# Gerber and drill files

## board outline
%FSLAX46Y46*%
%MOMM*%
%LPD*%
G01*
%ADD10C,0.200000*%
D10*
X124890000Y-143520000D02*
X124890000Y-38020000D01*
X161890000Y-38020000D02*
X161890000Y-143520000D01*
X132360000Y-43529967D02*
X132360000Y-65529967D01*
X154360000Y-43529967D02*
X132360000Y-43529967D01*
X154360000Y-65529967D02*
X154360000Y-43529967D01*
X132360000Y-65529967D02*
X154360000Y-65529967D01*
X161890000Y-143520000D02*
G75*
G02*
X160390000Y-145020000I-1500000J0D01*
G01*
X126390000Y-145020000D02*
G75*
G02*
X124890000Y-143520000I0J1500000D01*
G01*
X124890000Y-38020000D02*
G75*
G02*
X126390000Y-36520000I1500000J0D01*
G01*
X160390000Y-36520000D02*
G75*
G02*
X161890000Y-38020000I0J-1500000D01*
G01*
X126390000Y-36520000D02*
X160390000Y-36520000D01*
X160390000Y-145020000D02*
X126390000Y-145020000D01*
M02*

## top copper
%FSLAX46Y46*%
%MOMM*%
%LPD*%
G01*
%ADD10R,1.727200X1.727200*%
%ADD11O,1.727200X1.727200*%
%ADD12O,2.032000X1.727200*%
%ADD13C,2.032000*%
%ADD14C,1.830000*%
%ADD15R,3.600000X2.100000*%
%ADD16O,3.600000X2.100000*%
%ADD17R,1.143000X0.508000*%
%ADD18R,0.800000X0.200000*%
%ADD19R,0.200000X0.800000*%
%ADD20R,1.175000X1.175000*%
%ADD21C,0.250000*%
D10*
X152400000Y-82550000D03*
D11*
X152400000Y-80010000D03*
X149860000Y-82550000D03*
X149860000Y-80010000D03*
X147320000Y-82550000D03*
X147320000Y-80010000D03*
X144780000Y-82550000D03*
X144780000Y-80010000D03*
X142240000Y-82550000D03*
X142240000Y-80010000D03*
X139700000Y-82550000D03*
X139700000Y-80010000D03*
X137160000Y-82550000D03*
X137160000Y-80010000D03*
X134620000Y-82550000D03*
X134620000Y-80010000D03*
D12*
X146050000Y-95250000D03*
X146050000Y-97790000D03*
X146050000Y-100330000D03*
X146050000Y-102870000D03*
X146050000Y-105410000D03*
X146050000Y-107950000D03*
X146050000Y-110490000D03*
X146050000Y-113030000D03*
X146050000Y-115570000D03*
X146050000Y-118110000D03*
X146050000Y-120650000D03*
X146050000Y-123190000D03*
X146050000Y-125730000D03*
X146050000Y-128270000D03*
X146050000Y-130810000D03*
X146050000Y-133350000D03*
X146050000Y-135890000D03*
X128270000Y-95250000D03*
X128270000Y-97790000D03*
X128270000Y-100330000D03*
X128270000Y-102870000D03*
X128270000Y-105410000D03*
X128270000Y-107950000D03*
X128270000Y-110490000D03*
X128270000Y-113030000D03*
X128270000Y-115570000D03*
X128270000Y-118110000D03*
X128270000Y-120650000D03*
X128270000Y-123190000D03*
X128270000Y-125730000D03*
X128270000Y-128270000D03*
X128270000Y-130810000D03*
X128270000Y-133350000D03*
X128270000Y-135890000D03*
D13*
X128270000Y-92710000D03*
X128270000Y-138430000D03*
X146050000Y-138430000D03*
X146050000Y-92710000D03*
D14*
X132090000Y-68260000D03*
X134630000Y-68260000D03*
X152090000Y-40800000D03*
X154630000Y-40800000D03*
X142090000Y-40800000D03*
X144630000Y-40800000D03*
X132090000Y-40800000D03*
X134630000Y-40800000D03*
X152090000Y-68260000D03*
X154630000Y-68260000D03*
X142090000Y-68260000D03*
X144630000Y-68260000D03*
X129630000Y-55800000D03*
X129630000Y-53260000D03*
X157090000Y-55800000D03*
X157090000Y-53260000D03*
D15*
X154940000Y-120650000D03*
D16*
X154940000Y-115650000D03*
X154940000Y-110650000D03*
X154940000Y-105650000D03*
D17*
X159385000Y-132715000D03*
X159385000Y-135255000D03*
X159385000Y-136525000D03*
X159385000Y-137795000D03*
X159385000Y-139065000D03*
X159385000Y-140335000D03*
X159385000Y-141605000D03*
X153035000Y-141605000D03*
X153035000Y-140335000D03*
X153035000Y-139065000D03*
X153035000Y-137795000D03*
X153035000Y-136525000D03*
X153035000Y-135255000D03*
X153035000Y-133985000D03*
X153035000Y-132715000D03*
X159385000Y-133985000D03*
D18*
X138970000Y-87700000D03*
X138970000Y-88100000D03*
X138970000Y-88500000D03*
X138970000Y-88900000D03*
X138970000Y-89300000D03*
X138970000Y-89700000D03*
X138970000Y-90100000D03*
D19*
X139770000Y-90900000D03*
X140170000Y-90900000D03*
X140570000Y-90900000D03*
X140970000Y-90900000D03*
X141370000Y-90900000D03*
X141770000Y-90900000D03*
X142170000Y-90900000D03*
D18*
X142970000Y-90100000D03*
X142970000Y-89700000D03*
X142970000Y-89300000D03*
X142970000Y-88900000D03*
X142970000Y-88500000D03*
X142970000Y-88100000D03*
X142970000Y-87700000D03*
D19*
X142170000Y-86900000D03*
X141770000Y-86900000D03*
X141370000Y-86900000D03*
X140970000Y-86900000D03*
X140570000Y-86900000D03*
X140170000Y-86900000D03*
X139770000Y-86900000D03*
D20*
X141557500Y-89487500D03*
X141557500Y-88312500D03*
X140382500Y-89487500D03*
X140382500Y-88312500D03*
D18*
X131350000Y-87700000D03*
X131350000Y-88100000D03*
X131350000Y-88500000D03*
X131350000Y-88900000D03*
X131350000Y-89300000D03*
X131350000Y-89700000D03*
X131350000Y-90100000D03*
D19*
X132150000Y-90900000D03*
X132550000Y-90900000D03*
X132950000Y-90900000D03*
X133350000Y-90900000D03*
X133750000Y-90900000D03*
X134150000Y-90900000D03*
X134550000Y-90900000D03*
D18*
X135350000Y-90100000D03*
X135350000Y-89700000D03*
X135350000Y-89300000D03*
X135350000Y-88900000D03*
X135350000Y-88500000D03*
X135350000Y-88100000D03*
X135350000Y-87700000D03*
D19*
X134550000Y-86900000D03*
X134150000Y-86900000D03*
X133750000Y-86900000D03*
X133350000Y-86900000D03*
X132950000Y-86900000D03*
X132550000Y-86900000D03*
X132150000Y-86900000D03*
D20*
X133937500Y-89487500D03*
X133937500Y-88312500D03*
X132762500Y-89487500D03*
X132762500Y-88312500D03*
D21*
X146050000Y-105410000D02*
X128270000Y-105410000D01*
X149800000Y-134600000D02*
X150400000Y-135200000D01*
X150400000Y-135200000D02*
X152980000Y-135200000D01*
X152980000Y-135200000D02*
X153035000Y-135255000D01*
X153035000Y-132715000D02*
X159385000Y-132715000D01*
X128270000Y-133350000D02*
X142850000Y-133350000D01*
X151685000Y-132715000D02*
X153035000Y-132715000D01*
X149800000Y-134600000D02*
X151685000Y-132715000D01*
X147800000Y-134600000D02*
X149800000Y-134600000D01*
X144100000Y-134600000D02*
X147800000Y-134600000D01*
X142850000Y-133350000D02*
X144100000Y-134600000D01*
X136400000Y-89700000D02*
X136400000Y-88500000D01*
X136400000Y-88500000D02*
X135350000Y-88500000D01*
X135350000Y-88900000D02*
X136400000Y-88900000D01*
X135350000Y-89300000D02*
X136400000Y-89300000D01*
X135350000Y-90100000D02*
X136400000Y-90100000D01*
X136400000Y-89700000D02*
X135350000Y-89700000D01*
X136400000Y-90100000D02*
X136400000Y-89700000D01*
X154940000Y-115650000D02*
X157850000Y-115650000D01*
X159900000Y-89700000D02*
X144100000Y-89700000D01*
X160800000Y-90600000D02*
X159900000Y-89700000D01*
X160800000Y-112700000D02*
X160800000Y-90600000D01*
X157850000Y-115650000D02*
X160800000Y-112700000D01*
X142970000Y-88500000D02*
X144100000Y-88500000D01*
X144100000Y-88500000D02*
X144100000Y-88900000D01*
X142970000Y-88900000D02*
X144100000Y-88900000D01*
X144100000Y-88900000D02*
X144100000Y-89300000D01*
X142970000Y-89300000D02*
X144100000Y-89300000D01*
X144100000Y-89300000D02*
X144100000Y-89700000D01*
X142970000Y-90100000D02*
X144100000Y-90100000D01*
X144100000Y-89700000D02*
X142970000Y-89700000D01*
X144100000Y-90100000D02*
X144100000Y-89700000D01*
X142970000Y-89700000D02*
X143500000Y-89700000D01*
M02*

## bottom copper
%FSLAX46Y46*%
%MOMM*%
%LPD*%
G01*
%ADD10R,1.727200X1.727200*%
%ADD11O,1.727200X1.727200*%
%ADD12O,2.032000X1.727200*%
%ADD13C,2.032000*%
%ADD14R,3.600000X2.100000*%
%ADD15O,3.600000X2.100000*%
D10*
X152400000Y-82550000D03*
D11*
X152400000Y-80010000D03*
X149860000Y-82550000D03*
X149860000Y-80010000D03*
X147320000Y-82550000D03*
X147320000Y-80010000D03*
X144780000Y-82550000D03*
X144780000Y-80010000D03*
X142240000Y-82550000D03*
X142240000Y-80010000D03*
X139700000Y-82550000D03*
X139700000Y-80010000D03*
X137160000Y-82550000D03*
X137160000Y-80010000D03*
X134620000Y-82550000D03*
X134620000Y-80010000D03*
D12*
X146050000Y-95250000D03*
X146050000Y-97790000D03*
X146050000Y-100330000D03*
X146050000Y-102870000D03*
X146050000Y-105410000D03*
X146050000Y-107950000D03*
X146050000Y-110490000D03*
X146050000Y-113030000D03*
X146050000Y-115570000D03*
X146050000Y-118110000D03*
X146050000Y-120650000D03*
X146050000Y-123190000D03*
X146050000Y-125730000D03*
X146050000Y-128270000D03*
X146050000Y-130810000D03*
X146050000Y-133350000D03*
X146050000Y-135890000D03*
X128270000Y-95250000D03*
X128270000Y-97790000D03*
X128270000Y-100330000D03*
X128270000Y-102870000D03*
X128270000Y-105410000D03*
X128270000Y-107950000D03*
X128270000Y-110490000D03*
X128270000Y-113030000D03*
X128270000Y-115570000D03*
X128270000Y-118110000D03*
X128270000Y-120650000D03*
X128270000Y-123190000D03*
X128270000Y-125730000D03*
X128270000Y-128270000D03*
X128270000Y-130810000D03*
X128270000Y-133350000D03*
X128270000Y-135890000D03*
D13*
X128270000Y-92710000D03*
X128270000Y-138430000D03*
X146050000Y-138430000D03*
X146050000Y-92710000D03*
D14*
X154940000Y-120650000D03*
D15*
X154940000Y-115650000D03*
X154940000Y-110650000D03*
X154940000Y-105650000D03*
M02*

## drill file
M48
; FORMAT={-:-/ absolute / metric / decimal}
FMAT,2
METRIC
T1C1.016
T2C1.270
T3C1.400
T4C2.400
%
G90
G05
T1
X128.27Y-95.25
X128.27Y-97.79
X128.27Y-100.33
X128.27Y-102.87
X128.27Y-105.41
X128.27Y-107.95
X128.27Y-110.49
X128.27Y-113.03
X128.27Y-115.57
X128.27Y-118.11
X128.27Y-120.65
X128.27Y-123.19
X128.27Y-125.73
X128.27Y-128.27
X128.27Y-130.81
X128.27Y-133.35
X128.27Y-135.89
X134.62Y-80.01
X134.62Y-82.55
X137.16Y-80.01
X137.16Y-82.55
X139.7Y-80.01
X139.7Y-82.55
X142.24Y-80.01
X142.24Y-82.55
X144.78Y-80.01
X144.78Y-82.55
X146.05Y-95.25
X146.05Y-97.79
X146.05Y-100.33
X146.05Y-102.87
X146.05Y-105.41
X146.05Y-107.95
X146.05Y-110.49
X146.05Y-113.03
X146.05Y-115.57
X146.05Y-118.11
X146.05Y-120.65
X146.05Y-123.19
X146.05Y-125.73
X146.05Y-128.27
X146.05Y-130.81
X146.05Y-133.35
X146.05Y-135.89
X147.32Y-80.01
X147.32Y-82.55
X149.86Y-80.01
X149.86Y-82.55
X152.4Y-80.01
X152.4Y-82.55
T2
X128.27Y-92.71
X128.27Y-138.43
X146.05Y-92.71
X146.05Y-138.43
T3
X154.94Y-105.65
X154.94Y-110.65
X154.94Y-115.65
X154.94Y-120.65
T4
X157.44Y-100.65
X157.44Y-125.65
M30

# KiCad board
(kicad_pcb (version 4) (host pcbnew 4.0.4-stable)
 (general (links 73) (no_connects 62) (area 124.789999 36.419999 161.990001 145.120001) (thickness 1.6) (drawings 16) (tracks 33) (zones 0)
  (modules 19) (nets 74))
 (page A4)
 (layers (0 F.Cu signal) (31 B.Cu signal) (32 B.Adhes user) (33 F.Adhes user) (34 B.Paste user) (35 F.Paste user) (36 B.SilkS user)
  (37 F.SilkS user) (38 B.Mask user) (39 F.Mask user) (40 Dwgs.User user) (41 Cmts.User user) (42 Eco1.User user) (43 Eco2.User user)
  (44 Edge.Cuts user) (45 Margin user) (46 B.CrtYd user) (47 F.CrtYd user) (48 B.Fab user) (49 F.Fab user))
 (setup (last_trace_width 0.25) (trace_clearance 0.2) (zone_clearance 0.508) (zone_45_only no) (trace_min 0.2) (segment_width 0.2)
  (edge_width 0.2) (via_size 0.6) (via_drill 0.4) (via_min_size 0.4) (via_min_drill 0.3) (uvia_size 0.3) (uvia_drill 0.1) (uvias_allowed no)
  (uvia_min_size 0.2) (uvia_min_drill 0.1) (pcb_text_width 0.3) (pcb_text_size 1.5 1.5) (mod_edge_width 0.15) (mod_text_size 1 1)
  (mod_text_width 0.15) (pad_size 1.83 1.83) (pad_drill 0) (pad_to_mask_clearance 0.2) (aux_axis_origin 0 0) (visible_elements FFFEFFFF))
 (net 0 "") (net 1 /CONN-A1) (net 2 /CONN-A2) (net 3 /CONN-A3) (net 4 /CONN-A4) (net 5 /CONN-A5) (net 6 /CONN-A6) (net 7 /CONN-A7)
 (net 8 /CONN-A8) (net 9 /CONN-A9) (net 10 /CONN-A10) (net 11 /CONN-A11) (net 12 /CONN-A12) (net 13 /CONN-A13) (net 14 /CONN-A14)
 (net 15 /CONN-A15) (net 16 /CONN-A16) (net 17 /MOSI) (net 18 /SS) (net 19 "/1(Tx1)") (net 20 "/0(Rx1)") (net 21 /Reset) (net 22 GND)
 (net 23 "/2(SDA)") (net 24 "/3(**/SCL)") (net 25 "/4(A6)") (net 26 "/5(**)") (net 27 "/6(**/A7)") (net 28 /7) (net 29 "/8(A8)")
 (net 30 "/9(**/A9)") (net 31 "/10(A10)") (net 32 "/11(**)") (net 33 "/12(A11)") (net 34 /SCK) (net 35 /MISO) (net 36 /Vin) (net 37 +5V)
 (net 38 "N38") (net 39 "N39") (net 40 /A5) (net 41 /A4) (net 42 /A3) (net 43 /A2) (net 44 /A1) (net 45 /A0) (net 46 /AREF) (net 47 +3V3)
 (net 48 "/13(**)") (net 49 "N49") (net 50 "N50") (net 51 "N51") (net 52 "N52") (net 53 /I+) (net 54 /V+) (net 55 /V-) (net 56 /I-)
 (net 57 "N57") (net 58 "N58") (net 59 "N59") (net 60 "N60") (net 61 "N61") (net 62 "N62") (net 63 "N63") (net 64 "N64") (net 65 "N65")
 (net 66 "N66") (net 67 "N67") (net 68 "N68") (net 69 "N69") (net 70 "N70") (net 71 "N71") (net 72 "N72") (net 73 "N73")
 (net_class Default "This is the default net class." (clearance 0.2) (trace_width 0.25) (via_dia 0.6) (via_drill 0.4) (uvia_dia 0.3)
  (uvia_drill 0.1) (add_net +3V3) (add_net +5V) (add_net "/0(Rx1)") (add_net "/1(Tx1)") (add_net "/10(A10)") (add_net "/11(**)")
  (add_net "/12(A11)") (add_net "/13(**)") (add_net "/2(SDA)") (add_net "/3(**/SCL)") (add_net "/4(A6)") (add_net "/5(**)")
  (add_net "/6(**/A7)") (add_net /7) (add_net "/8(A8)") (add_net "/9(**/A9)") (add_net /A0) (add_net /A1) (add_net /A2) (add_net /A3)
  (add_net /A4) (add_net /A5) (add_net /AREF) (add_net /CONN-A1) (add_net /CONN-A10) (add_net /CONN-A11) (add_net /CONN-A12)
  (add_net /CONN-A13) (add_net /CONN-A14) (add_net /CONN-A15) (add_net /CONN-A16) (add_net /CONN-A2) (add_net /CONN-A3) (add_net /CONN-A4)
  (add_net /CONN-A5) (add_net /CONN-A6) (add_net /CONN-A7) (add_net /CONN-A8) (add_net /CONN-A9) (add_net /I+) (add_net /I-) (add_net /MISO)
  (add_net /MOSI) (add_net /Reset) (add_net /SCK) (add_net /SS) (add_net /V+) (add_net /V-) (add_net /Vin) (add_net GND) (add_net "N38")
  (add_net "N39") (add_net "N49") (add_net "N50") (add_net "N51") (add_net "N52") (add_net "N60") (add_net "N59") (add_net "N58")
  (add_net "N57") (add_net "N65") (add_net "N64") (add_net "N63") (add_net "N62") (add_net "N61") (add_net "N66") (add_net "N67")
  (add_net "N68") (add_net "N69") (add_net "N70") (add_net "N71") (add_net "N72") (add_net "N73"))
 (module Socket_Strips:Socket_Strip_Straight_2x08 (layer F.Cu) (at 152.4 82.55 180)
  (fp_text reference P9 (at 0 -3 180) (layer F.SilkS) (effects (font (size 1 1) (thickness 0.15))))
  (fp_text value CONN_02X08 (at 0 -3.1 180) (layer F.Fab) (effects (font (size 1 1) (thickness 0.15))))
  (pad 1 thru_hole rect (at 0 0 180) (size 1.7272 1.7272) (drill 1.016) (layers *.Cu *.Mask F.SilkS) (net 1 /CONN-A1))
  (pad 2 thru_hole oval (at 0 2.54 180) (size 1.7272 1.7272) (drill 1.016) (layers *.Cu *.Mask F.SilkS) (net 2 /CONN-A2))
  (pad 3 thru_hole oval (at 2.54 0 180) (size 1.7272 1.7272) (drill 1.016) (layers *.Cu *.Mask F.SilkS) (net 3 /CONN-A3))
  (pad 4 thru_hole oval (at 2.54 2.54 180) (size 1.7272 1.7272) (drill 1.016) (layers *.Cu *.Mask F.SilkS) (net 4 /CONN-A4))
  (pad 5 thru_hole oval (at 5.08 0 180) (size 1.7272 1.7272) (drill 1.016) (layers *.Cu *.Mask F.SilkS) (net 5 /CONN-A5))
  (pad 6 thru_hole oval (at 5.08 2.54 180) (size 1.7272 1.7272) (drill 1.016) (layers *.Cu *.Mask F.SilkS) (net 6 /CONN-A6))
  (pad 7 thru_hole oval (at 7.62 0 180) (size 1.7272 1.7272) (drill 1.016) (layers *.Cu *.Mask F.SilkS) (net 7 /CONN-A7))
  (pad 8 thru_hole oval (at 7.62 2.54 180) (size 1.7272 1.7272) (drill 1.016) (layers *.Cu *.Mask F.SilkS) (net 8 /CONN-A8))
  (pad 9 thru_hole oval (at 10.16 0 180) (size 1.7272 1.7272) (drill 1.016) (layers *.Cu *.Mask F.SilkS) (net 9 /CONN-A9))
  (pad 10 thru_hole oval (at 10.16 2.54 180) (size 1.7272 1.7272) (drill 1.016) (layers *.Cu *.Mask F.SilkS) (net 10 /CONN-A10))
  (pad 11 thru_hole oval (at 12.7 0 180) (size 1.7272 1.7272) (drill 1.016) (layers *.Cu *.Mask F.SilkS) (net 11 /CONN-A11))
  (pad 12 thru_hole oval (at 12.7 2.54 180) (size 1.7272 1.7272) (drill 1.016) (layers *.Cu *.Mask F.SilkS) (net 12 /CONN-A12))
  (pad 13 thru_hole oval (at 15.24 0 180) (size 1.7272 1.7272) (drill 1.016) (layers *.Cu *.Mask F.SilkS) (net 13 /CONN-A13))
  (pad 14 thru_hole oval (at 15.24 2.54 180) (size 1.7272 1.7272) (drill 1.016) (layers *.Cu *.Mask F.SilkS) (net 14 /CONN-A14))
  (pad 15 thru_hole oval (at 17.78 0 180) (size 1.7272 1.7272) (drill 1.016) (layers *.Cu *.Mask F.SilkS) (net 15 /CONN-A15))
  (pad 16 thru_hole oval (at 17.78 2.54 180) (size 1.7272 1.7272) (drill 1.016) (layers *.Cu *.Mask F.SilkS) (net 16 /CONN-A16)))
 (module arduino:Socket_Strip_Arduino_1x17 (layer F.Cu) (at 146.05 95.25 270)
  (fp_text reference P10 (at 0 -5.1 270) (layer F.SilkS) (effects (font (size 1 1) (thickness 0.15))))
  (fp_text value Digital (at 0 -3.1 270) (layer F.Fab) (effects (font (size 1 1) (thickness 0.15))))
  (pad 1 thru_hole oval (at 0 0 270) (size 1.7272 2.032) (drill 1.016) (layers *.Cu *.Mask F.SilkS) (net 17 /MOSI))
  (pad 2 thru_hole oval (at 2.54 0 270) (size 1.7272 2.032) (drill 1.016) (layers *.Cu *.Mask F.SilkS) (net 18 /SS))
  (pad 3 thru_hole oval (at 5.08 0 270) (size 1.7272 2.032) (drill 1.016) (layers *.Cu *.Mask F.SilkS) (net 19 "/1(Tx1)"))
  (pad 4 thru_hole oval (at 7.62 0 270) (size 1.7272 2.032) (drill 1.016) (layers *.Cu *.Mask F.SilkS) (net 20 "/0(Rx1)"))
  (pad 5 thru_hole oval (at 10.16 0 270) (size 1.7272 2.032) (drill 1.016) (layers *.Cu *.Mask F.SilkS) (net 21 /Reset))
  (pad 6 thru_hole oval (at 12.7 0 270) (size 1.7272 2.032) (drill 1.016) (layers *.Cu *.Mask F.SilkS) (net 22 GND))
  (pad 7 thru_hole oval (at 15.24 0 270) (size 1.7272 2.032) (drill 1.016) (layers *.Cu *.Mask F.SilkS) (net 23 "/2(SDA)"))
  (pad 8 thru_hole oval (at 17.78 0 270) (size 1.7272 2.032) (drill 1.016) (layers *.Cu *.Mask F.SilkS) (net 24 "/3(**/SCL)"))
  (pad 9 thru_hole oval (at 20.32 0 270) (size 1.7272 2.032) (drill 1.016) (layers *.Cu *.Mask F.SilkS) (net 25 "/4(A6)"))
  (pad 10 thru_hole oval (at 22.86 0 270) (size 1.7272 2.032) (drill 1.016) (layers *.Cu *.Mask F.SilkS) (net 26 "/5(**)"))
  (pad 11 thru_hole oval (at 25.4 0 270) (size 1.7272 2.032) (drill 1.016) (layers *.Cu *.Mask F.SilkS) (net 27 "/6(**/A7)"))
  (pad 12 thru_hole oval (at 27.94 0 270) (size 1.7272 2.032) (drill 1.016) (layers *.Cu *.Mask F.SilkS) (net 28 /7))
  (pad 13 thru_hole oval (at 30.48 0 270) (size 1.7272 2.032) (drill 1.016) (layers *.Cu *.Mask F.SilkS) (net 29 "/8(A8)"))
  (pad 14 thru_hole oval (at 33.02 0 270) (size 1.7272 2.032) (drill 1.016) (layers *.Cu *.Mask F.SilkS) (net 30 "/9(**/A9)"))
  (pad 15 thru_hole oval (at 35.56 0 270) (size 1.7272 2.032) (drill 1.016) (layers *.Cu *.Mask F.SilkS) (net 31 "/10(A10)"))
  (pad 16 thru_hole oval (at 38.1 0 270) (size 1.7272 2.032) (drill 1.016) (layers *.Cu *.Mask F.SilkS) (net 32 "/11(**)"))
  (pad 17 thru_hole oval (at 40.64 0 270) (size 1.7272 2.032) (drill 1.016) (layers *.Cu *.Mask F.SilkS) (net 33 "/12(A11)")))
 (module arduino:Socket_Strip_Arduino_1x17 (layer F.Cu) (at 128.27 95.25 270)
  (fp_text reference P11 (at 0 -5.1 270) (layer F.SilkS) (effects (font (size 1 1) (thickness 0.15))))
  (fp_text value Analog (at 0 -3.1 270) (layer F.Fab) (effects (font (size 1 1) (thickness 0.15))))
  (pad 1 thru_hole oval (at 0 0 270) (size 1.7272 2.032) (drill 1.016) (layers *.Cu *.Mask F.SilkS) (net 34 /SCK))
  (pad 2 thru_hole oval (at 2.54 0 270) (size 1.7272 2.032) (drill 1.016) (layers *.Cu *.Mask F.SilkS) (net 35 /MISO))
  (pad 3 thru_hole oval (at 5.08 0 270) (size 1.7272 2.032) (drill 1.016) (layers *.Cu *.Mask F.SilkS) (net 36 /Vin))
  (pad 4 thru_hole oval (at 7.62 0 270) (size 1.7272 2.032) (drill 1.016) (layers *.Cu *.Mask F.SilkS) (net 22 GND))
  (pad 5 thru_hole oval (at 10.16 0 270) (size 1.7272 2.032) (drill 1.016) (layers *.Cu *.Mask F.SilkS) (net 21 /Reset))
  (pad 6 thru_hole oval (at 12.7 0 270) (size 1.7272 2.032) (drill 1.016) (layers *.Cu *.Mask F.SilkS) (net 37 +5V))
  (pad 7 thru_hole oval (at 15.24 0 270) (size 1.7272 2.032) (drill 1.016) (layers *.Cu *.Mask F.SilkS) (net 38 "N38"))
  (pad 8 thru_hole oval (at 17.78 0 270) (size 1.7272 2.032) (drill 1.016) (layers *.Cu *.Mask F.SilkS) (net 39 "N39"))
  (pad 9 thru_hole oval (at 20.32 0 270) (size 1.7272 2.032) (drill 1.016) (layers *.Cu *.Mask F.SilkS) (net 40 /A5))
  (pad 10 thru_hole oval (at 22.86 0 270) (size 1.7272 2.032) (drill 1.016) (layers *.Cu *.Mask F.SilkS) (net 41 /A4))
  (pad 11 thru_hole oval (at 25.4 0 270) (size 1.7272 2.032) (drill 1.016) (layers *.Cu *.Mask F.SilkS) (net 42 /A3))
  (pad 12 thru_hole oval (at 27.94 0 270) (size 1.7272 2.032) (drill 1.016) (layers *.Cu *.Mask F.SilkS) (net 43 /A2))
  (pad 13 thru_hole oval (at 30.48 0 270) (size 1.7272 2.032) (drill 1.016) (layers *.Cu *.Mask F.SilkS) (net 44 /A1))
  (pad 14 thru_hole oval (at 33.02 0 270) (size 1.7272 2.032) (drill 1.016) (layers *.Cu *.Mask F.SilkS) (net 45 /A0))
  (pad 15 thru_hole oval (at 35.56 0 270) (size 1.7272 2.032) (drill 1.016) (layers *.Cu *.Mask F.SilkS) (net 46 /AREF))
  (pad 16 thru_hole oval (at 38.1 0 270) (size 1.7272 2.032) (drill 1.016) (layers *.Cu *.Mask F.SilkS) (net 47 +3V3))
  (pad 17 thru_hole oval (at 40.64 0 270) (size 1.7272 2.032) (drill 1.016) (layers *.Cu *.Mask F.SilkS) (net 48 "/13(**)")))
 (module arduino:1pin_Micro (layer F.Cu) (at 128.27 92.71)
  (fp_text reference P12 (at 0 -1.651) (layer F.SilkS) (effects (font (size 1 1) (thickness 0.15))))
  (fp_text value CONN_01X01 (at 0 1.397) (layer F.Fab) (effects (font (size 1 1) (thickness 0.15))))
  (pad 1 thru_hole circle (at 0 0) (size 2.032 2.032) (drill 1.27) (layers *.Cu *.Mask F.SilkS) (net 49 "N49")))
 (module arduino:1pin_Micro (layer F.Cu) (at 128.27 138.43)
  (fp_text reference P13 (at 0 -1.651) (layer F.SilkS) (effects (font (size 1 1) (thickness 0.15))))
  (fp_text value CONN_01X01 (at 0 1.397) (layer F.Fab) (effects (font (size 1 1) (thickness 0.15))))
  (pad 1 thru_hole circle (at 0 0) (size 2.032 2.032) (drill 1.27) (layers *.Cu *.Mask F.SilkS) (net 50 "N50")))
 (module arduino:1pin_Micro (layer F.Cu) (at 146.05 138.43)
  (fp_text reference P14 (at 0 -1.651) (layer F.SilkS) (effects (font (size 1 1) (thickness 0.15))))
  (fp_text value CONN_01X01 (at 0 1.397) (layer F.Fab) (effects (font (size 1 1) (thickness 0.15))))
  (pad 1 thru_hole circle (at 0 0) (size 2.032 2.032) (drill 1.27) (layers *.Cu *.Mask F.SilkS) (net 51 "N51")))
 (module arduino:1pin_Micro (layer F.Cu) (at 146.05 92.71)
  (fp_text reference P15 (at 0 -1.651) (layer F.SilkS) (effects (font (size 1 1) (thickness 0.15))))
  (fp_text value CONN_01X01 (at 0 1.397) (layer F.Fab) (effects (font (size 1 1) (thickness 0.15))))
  (pad 1 thru_hole circle (at 0 0) (size 2.032 2.032) (drill 1.27) (layers *.Cu *.Mask F.SilkS) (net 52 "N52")))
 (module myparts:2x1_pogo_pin (layer F.Cu) (at 132.09 68.26)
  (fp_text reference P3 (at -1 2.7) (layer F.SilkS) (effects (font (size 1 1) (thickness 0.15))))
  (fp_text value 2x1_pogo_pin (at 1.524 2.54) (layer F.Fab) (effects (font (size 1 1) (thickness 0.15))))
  (pad 1 smd circle (at 0 0) (size 1.83 1.83) (layers F.Cu F.Paste F.Mask) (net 13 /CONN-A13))
  (pad 2 smd circle (at 2.54 0) (size 1.83 1.83) (layers F.Cu F.Paste F.Mask) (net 14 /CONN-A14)))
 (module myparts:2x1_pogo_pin (layer F.Cu) (at 152.09 40.8)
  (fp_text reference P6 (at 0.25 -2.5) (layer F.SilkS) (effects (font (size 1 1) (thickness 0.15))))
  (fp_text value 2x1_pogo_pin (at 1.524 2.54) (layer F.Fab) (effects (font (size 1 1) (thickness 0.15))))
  (pad 1 smd circle (at 0 0) (size 1.83 1.83) (layers F.Cu F.Paste F.Mask) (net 5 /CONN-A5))
  (pad 2 smd circle (at 2.54 0) (size 1.83 1.83) (layers F.Cu F.Paste F.Mask) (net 6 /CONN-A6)))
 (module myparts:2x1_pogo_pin (layer F.Cu) (at 142.09 40.8)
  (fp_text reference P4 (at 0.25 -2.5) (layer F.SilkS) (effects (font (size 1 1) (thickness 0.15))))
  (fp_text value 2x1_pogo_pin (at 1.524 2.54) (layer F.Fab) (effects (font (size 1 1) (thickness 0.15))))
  (pad 1 smd circle (at 0 0) (size 1.83 1.83) (layers F.Cu F.Paste F.Mask) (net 7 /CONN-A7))
  (pad 2 smd circle (at 2.54 0) (size 1.83 1.83) (layers F.Cu F.Paste F.Mask) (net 8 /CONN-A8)))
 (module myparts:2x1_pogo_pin (layer F.Cu) (at 132.09 40.8)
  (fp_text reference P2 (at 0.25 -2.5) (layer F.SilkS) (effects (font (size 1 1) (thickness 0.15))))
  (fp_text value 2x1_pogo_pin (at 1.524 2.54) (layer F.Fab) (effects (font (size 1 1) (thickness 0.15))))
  (pad 1 smd circle (at 0 0) (size 1.83 1.83) (layers F.Cu F.Paste F.Mask) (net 11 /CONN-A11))
  (pad 2 smd circle (at 2.54 0) (size 1.83 1.83) (layers F.Cu F.Paste F.Mask) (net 12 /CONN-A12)))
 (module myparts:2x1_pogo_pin (layer F.Cu) (at 152.09 68.26)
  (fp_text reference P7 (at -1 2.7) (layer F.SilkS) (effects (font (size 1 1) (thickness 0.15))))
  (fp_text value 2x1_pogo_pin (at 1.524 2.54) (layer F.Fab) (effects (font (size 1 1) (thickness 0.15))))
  (pad 1 smd circle (at 0 0) (size 1.83 1.83) (layers F.Cu F.Paste F.Mask) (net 3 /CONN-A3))
  (pad 2 smd circle (at 2.54 0) (size 1.83 1.83) (layers F.Cu F.Paste F.Mask) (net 4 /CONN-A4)))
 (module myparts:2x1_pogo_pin (layer F.Cu) (at 142.09 68.26)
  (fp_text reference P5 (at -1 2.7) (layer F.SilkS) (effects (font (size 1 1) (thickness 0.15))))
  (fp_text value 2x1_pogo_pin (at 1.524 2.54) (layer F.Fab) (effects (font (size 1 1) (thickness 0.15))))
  (pad 1 smd circle (at 0 0) (size 1.83 1.83) (layers F.Cu F.Paste F.Mask) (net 9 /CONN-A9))
  (pad 2 smd circle (at 2.54 0) (size 1.83 1.83) (layers F.Cu F.Paste F.Mask) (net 10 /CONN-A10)))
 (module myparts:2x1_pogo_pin (layer F.Cu) (at 129.63 55.8 90)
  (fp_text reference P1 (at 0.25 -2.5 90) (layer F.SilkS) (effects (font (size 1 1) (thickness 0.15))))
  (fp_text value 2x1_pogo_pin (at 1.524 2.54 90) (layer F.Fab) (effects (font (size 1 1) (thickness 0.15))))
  (pad 1 smd circle (at 0 0 90) (size 1.83 1.83) (layers F.Cu F.Paste F.Mask) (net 15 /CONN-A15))
  (pad 2 smd circle (at 2.54 0 90) (size 1.83 1.83) (layers F.Cu F.Paste F.Mask) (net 16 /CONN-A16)))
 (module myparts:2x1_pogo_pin (layer F.Cu) (at 157.09 55.8 90)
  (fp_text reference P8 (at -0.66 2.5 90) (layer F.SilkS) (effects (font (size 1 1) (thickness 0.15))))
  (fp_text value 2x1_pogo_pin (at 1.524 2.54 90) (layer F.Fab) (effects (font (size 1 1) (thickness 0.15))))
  (pad 1 smd circle (at 0 0 90) (size 1.83 1.83) (layers F.Cu F.Paste F.Mask) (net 1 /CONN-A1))
  (pad 2 smd circle (at 2.54 0 90) (size 1.83 1.83) (layers F.Cu F.Paste F.Mask) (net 2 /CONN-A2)))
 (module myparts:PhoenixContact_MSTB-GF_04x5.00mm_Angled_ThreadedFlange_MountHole (layer F.Cu) (at 154.94 120.65 90)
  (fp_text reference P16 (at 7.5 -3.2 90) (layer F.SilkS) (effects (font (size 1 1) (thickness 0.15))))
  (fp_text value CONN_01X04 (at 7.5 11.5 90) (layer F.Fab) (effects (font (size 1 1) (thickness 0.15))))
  (pad 1 thru_hole rect (at 0 0 90) (size 2.1 3.6) (drill 1.4) (layers *.Cu *.Mask) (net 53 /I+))
  (pad 2 thru_hole oval (at 5 0 90) (size 2.1 3.6) (drill 1.4) (layers *.Cu *.Mask) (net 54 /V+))
  (pad 3 thru_hole oval (at 10 0 90) (size 2.1 3.6) (drill 1.4) (layers *.Cu *.Mask) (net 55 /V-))
  (pad 4 thru_hole oval (at 15 0 90) (size 2.1 3.6) (drill 1.4) (layers *.Cu *.Mask) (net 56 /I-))
  (pad "" np_thru_hole circle (at -5 2.5 90) (size 2.4 2.4) (drill 2.4) (layers *.Cu *.Mask))
  (pad "" np_thru_hole circle (at 20 2.5 90) (size 2.4 2.4) (drill 2.4) (layers *.Cu *.Mask)))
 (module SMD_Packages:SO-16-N (layer F.Cu) (at 156.21 137.16 270)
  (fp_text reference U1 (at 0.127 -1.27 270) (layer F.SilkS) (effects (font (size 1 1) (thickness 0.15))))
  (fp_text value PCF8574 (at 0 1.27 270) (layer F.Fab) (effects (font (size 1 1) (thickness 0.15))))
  (pad 16 smd rect (at -4.445 -3.175 270) (size 0.508 1.143) (layers F.Cu F.Paste F.Mask) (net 47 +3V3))
  (pad 14 smd rect (at -1.905 -3.175 270) (size 0.508 1.143) (layers F.Cu F.Paste F.Mask) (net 24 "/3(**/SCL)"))
  (pad 13 smd rect (at -0.635 -3.175 270) (size 0.508 1.143) (layers F.Cu F.Paste F.Mask) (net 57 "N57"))
  (pad 12 smd rect (at 0.635 -3.175 270) (size 0.508 1.143) (layers F.Cu F.Paste F.Mask) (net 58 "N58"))
  (pad 11 smd rect (at 1.905 -3.175 270) (size 0.508 1.143) (layers F.Cu F.Paste F.Mask) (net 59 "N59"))
  (pad 10 smd rect (at 3.175 -3.175 270) (size 0.508 1.143) (layers F.Cu F.Paste F.Mask) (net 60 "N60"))
  (pad 9 smd rect (at 4.445 -3.175 270) (size 0.508 1.143) (layers F.Cu F.Paste F.Mask) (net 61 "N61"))
  (pad 8 smd rect (at 4.445 3.175 270) (size 0.508 1.143) (layers F.Cu F.Paste F.Mask) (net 22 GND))
  (pad 7 smd rect (at 3.175 3.175 270) (size 0.508 1.143) (layers F.Cu F.Paste F.Mask) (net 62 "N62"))
  (pad 6 smd rect (at 1.905 3.175 270) (size 0.508 1.143) (layers F.Cu F.Paste F.Mask) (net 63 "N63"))
  (pad 5 smd rect (at 0.635 3.175 270) (size 0.508 1.143) (layers F.Cu F.Paste F.Mask) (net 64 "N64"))
  (pad 4 smd rect (at -0.635 3.175 270) (size 0.508 1.143) (layers F.Cu F.Paste F.Mask) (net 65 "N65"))
  (pad 3 smd rect (at -1.905 3.175 270) (size 0.508 1.143) (layers F.Cu F.Paste F.Mask) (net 47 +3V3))
  (pad 2 smd rect (at -3.175 3.175 270) (size 0.508 1.143) (layers F.Cu F.Paste F.Mask) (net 22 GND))
  (pad 1 smd rect (at -4.445 3.175 270) (size 0.508 1.143) (layers F.Cu F.Paste F.Mask) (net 47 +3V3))
  (pad 15 smd rect (at -3.175 -3.175 270) (size 0.508 1.143) (layers F.Cu F.Paste F.Mask) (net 23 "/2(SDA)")))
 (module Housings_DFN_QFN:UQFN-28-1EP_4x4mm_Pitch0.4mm (layer F.Cu) (at 140.97 88.9)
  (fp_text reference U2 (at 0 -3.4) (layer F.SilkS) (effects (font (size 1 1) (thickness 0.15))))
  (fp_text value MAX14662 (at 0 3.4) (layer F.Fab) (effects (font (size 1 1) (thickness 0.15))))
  (pad 1 smd rect (at -2 -1.2) (size 0.8 0.2) (layers F.Cu F.Paste F.Mask) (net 47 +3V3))
  (pad 2 smd rect (at -2 -0.8) (size 0.8 0.2) (layers F.Cu F.Paste F.Mask) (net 16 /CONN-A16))
  (pad 3 smd rect (at -2 -0.4) (size 0.8 0.2) (layers F.Cu F.Paste F.Mask) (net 14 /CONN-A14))
  (pad 4 smd rect (at -2 0) (size 0.8 0.2) (layers F.Cu F.Paste F.Mask) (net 12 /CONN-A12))
  (pad 5 smd rect (at -2 0.4) (size 0.8 0.2) (layers F.Cu F.Paste F.Mask) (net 10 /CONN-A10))
  (pad 6 smd rect (at -2 0.8) (size 0.8 0.2) (layers F.Cu F.Paste F.Mask) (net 8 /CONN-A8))
  (pad 7 smd rect (at -2 1.2) (size 0.8 0.2) (layers F.Cu F.Paste F.Mask) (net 6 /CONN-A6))
  (pad 8 smd rect (at -1.2 2 90) (size 0.8 0.2) (layers F.Cu F.Paste F.Mask) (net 4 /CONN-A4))
  (pad 9 smd rect (at -0.8 2 90) (size 0.8 0.2) (layers F.Cu F.Paste F.Mask) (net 2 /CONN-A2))
  (pad 10 smd rect (at -0.4 2 90) (size 0.8 0.2) (layers F.Cu F.Paste F.Mask) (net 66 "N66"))
  (pad 11 smd rect (at 0 2 90) (size 0.8 0.2) (layers F.Cu F.Paste F.Mask) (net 22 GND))
  (pad 12 smd rect (at 0.4 2 90) (size 0.8 0.2) (layers F.Cu F.Paste F.Mask) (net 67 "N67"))
  (pad 13 smd rect (at 0.8 2 90) (size 0.8 0.2) (layers F.Cu F.Paste F.Mask) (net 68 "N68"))
  (pad 14 smd rect (at 1.2 2 90) (size 0.8 0.2) (layers F.Cu F.Paste F.Mask) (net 55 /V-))
  (pad 15 smd rect (at 2 1.2) (size 0.8 0.2) (layers F.Cu F.Paste F.Mask) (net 54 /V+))
  (pad 16 smd rect (at 2 0.8) (size 0.8 0.2) (layers F.Cu F.Paste F.Mask) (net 54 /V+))
  (pad 17 smd rect (at 2 0.4) (size 0.8 0.2) (layers F.Cu F.Paste F.Mask) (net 54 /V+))
  (pad 18 smd rect (at 2 0) (size 0.8 0.2) (layers F.Cu F.Paste F.Mask) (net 54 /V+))
  (pad 19 smd rect (at 2 -0.4) (size 0.8 0.2) (layers F.Cu F.Paste F.Mask) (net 54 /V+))
  (pad 20 smd rect (at 2 -0.8) (size 0.8 0.2) (layers F.Cu F.Paste F.Mask) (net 54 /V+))
  (pad 21 smd rect (at 2 -1.2) (size 0.8 0.2) (layers F.Cu F.Paste F.Mask) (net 55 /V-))
  (pad 22 smd rect (at 1.2 -2 90) (size 0.8 0.2) (layers F.Cu F.Paste F.Mask) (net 47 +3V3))
  (pad 23 smd rect (at 0.8 -2 90) (size 0.8 0.2) (layers F.Cu F.Paste F.Mask) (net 65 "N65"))
  (pad 24 smd rect (at 0.4 -2 90) (size 0.8 0.2) (layers F.Cu F.Paste F.Mask) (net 34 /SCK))
  (pad 25 smd rect (at 0 -2 90) (size 0.8 0.2) (layers F.Cu F.Paste F.Mask) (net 22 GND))
  (pad 26 smd rect (at -0.4 -2 90) (size 0.8 0.2) (layers F.Cu F.Paste F.Mask) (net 47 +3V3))
  (pad 27 smd rect (at -0.8 -2 90) (size 0.8 0.2) (layers F.Cu F.Paste F.Mask) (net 17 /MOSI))
  (pad 28 smd rect (at -1.2 -2 90) (size 0.8 0.2) (layers F.Cu F.Paste F.Mask) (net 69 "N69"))
  (pad 29 smd rect (at 0.5875 0.5875) (size 1.175 1.175) (layers F.Cu F.Paste F.Mask) (solder_paste_margin_ratio -0.2))
  (pad 29 smd rect (at 0.5875 -0.5875) (size 1.175 1.175) (layers F.Cu F.Paste F.Mask) (solder_paste_margin_ratio -0.2))
  (pad 29 smd rect (at -0.5875 0.5875) (size 1.175 1.175) (layers F.Cu F.Paste F.Mask) (solder_paste_margin_ratio -0.2))
  (pad 29 smd rect (at -0.5875 -0.5875) (size 1.175 1.175) (layers F.Cu F.Paste F.Mask) (solder_paste_margin_ratio -0.2)))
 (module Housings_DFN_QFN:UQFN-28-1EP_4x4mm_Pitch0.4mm (layer F.Cu) (at 133.35 88.9)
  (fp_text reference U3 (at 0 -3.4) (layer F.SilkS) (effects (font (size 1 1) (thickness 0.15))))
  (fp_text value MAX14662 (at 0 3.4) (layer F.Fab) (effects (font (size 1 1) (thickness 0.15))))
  (pad 1 smd rect (at -2 -1.2) (size 0.8 0.2) (layers F.Cu F.Paste F.Mask) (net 47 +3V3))
  (pad 2 smd rect (at -2 -0.8) (size 0.8 0.2) (layers F.Cu F.Paste F.Mask) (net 15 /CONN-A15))
  (pad 3 smd rect (at -2 -0.4) (size 0.8 0.2) (layers F.Cu F.Paste F.Mask) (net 13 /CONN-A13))
  (pad 4 smd rect (at -2 0) (size 0.8 0.2) (layers F.Cu F.Paste F.Mask) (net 11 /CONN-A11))
  (pad 5 smd rect (at -2 0.4) (size 0.8 0.2) (layers F.Cu F.Paste F.Mask) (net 9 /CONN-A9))
  (pad 6 smd rect (at -2 0.8) (size 0.8 0.2) (layers F.Cu F.Paste F.Mask) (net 7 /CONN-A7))
  (pad 7 smd rect (at -2 1.2) (size 0.8 0.2) (layers F.Cu F.Paste F.Mask) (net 5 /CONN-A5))
  (pad 8 smd rect (at -1.2 2 90) (size 0.8 0.2) (layers F.Cu F.Paste F.Mask) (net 3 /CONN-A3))
  (pad 9 smd rect (at -0.8 2 90) (size 0.8 0.2) (layers F.Cu F.Paste F.Mask) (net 1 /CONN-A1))
  (pad 10 smd rect (at -0.4 2 90) (size 0.8 0.2) (layers F.Cu F.Paste F.Mask) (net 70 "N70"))
  (pad 11 smd rect (at 0 2 90) (size 0.8 0.2) (layers F.Cu F.Paste F.Mask) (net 22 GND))
  (pad 12 smd rect (at 0.4 2 90) (size 0.8 0.2) (layers F.Cu F.Paste F.Mask) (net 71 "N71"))
  (pad 13 smd rect (at 0.8 2 90) (size 0.8 0.2) (layers F.Cu F.Paste F.Mask) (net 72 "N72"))
  (pad 14 smd rect (at 1.2 2 90) (size 0.8 0.2) (layers F.Cu F.Paste F.Mask) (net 56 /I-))
  (pad 15 smd rect (at 2 1.2) (size 0.8 0.2) (layers F.Cu F.Paste F.Mask) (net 53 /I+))
  (pad 16 smd rect (at 2 0.8) (size 0.8 0.2) (layers F.Cu F.Paste F.Mask) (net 53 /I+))
  (pad 17 smd rect (at 2 0.4) (size 0.8 0.2) (layers F.Cu F.Paste F.Mask) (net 53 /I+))
  (pad 18 smd rect (at 2 0) (size 0.8 0.2) (layers F.Cu F.Paste F.Mask) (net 53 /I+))
  (pad 19 smd rect (at 2 -0.4) (size 0.8 0.2) (layers F.Cu F.Paste F.Mask) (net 53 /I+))
  (pad 20 smd rect (at 2 -0.8) (size 0.8 0.2) (layers F.Cu F.Paste F.Mask) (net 53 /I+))
  (pad 21 smd rect (at 2 -1.2) (size 0.8 0.2) (layers F.Cu F.Paste F.Mask) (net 56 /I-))
  (pad 22 smd rect (at 1.2 -2 90) (size 0.8 0.2) (layers F.Cu F.Paste F.Mask) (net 47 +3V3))
  (pad 23 smd rect (at 0.8 -2 90) (size 0.8 0.2) (layers F.Cu F.Paste F.Mask) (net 69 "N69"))
  (pad 24 smd rect (at 0.4 -2 90) (size 0.8 0.2) (layers F.Cu F.Paste F.Mask) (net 34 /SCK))
  (pad 25 smd rect (at 0 -2 90) (size 0.8 0.2) (layers F.Cu F.Paste F.Mask) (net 22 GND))
  (pad 26 smd rect (at -0.4 -2 90) (size 0.8 0.2) (layers F.Cu F.Paste F.Mask) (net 47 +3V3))
  (pad 27 smd rect (at -0.8 -2 90) (size 0.8 0.2) (layers F.Cu F.Paste F.Mask) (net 17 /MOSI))
  (pad 28 smd rect (at -1.2 -2 90) (size 0.8 0.2) (layers F.Cu F.Paste F.Mask) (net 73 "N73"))
  (pad 29 smd rect (at 0.5875 0.5875) (size 1.175 1.175) (layers F.Cu F.Paste F.Mask) (solder_paste_margin_ratio -0.2))
  (pad 29 smd rect (at 0.5875 -0.5875) (size 1.175 1.175) (layers F.Cu F.Paste F.Mask) (solder_paste_margin_ratio -0.2))
  (pad 29 smd rect (at -0.5875 0.5875) (size 1.175 1.175) (layers F.Cu F.Paste F.Mask) (solder_paste_margin_ratio -0.2))
  (pad 29 smd rect (at -0.5875 -0.5875) (size 1.175 1.175) (layers F.Cu F.Paste F.Mask) (solder_paste_margin_ratio -0.2)))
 (gr_line (start 124.89 143.52) (end 124.89 38.02) (angle 90) (layer Edge.Cuts) (width 0.2))
 (gr_line (start 161.89 38.02) (end 161.89 143.52) (angle 90) (layer Edge.Cuts) (width 0.2))
 (gr_line (start 132.36 43.529967) (end 132.36 65.529967) (layer Edge.Cuts) (width 0.2))
 (gr_line (start 154.36 43.529967) (end 132.36 43.529967) (layer Edge.Cuts) (width 0.2))
 (gr_line (start 154.36 65.529967) (end 154.36 43.529967) (layer Edge.Cuts) (width 0.2))
 (gr_line (start 132.36 65.529967) (end 154.36 65.529967) (layer Edge.Cuts) (width 0.2))
 (gr_arc (start 160.39 143.52) (end 161.89 143.52) (angle 90) (layer Edge.Cuts) (width 0.2))
 (gr_arc (start 126.39 143.52) (end 126.39 145.02) (angle 90) (layer Edge.Cuts) (width 0.2))
 (gr_arc (start 126.39 38.02) (end 124.89 38.02) (angle 90) (layer Edge.Cuts) (width 0.2))
 (gr_arc (start 160.39 38.02) (end 160.39 36.52) (angle 90) (layer Edge.Cuts) (width 0.2))
 (gr_line (start 126.39 36.52) (end 160.39 36.52) (angle 90) (layer Edge.Cuts) (width 0.2))
 (gr_line (start 160.39 145.02) (end 126.39 145.02) (angle 90) (layer Edge.Cuts) (width 0.2))
 (segment (start 146.05 105.41) (end 128.27 105.41) (width 0.25) (layer F.Cu) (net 21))
 (segment (start 149.8 134.6) (end 150.4 135.2) (width 0.25) (layer F.Cu) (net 47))
 (segment (start 150.4 135.2) (end 152.98 135.2) (width 0.25) (layer F.Cu) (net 47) (status 800000))
 (segment (start 152.98 135.2) (end 153.035 135.255) (width 0.25) (layer F.Cu) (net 47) (status C00000))
 (segment (start 153.035 132.715) (end 159.385 132.715) (width 0.25) (layer F.Cu) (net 47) (status C00000))
 (segment (start 128.27 133.35) (end 142.85 133.35) (width 0.25) (layer F.Cu) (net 47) (status 400000))
 (segment (start 151.685 132.715) (end 153.035 132.715) (width 0.25) (layer F.Cu) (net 47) (status 800000))
 (segment (start 149.8 134.6) (end 151.685 132.715) (width 0.25) (layer F.Cu) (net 47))
 (segment (start 147.8 134.6) (end 149.8 134.6) (width 0.25) (layer F.Cu) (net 47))
 (segment (start 144.1 134.6) (end 147.8 134.6) (width 0.25) (layer F.Cu) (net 47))
 (segment (start 142.85 133.35) (end 144.1 134.6) (width 0.25) (layer F.Cu) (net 47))
 (segment (start 136.4 89.7) (end 136.4 88.5) (width 0.25) (layer F.Cu) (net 53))
 (segment (start 136.4 88.5) (end 135.35 88.5) (width 0.25) (layer F.Cu) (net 53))
 (segment (start 135.35 88.9) (end 136.4 88.9) (width 0.25) (layer F.Cu) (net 53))
 (segment (start 135.35 89.3) (end 136.4 89.3) (width 0.25) (layer F.Cu) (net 53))
 (segment (start 135.35 90.1) (end 136.4 90.1) (width 0.25) (layer F.Cu) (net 53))
 (segment (start 136.4 89.7) (end 135.35 89.7) (width 0.25) (layer F.Cu) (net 53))
 (segment (start 136.4 90.1) (end 136.4 89.7) (width 0.25) (layer F.Cu) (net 53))
 (segment (start 154.94 115.65) (end 157.85 115.65) (width 0.25) (layer F.Cu) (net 54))
 (segment (start 159.9 89.7) (end 144.1 89.7) (width 0.25) (layer F.Cu) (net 54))
 (segment (start 160.8 90.6) (end 159.9 89.7) (width 0.25) (layer F.Cu) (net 54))
 (segment (start 160.8 112.7) (end 160.8 90.6) (width 0.25) (layer F.Cu) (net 54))
 (segment (start 157.85 115.65) (end 160.8 112.7) (width 0.25) (layer F.Cu) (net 54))
 (segment (start 142.97 88.5) (end 144.1 88.5) (width 0.25) (layer F.Cu) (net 54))
 (segment (start 144.1 88.5) (end 144.1 88.9) (width 0.25) (layer F.Cu) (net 54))
 (segment (start 142.97 88.9) (end 144.1 88.9) (width 0.25) (layer F.Cu) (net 54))
 (segment (start 144.1 88.9) (end 144.1 89.3) (width 0.25) (layer F.Cu) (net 54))
 (segment (start 142.97 89.3) (end 144.1 89.3) (width 0.25) (layer F.Cu) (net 54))
 (segment (start 144.1 89.3) (end 144.1 89.7) (width 0.25) (layer F.Cu) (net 54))
 (segment (start 142.97 90.1) (end 144.1 90.1) (width 0.25) (layer F.Cu) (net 54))
 (segment (start 144.1 89.7) (end 142.97 89.7) (width 0.25) (layer F.Cu) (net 54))
 (segment (start 144.1 90.1) (end 144.1 89.7) (width 0.25) (layer F.Cu) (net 54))
 (segment (start 142.97 89.7) (end 143.5 89.7) (width 0.25) (layer F.Cu) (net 54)))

